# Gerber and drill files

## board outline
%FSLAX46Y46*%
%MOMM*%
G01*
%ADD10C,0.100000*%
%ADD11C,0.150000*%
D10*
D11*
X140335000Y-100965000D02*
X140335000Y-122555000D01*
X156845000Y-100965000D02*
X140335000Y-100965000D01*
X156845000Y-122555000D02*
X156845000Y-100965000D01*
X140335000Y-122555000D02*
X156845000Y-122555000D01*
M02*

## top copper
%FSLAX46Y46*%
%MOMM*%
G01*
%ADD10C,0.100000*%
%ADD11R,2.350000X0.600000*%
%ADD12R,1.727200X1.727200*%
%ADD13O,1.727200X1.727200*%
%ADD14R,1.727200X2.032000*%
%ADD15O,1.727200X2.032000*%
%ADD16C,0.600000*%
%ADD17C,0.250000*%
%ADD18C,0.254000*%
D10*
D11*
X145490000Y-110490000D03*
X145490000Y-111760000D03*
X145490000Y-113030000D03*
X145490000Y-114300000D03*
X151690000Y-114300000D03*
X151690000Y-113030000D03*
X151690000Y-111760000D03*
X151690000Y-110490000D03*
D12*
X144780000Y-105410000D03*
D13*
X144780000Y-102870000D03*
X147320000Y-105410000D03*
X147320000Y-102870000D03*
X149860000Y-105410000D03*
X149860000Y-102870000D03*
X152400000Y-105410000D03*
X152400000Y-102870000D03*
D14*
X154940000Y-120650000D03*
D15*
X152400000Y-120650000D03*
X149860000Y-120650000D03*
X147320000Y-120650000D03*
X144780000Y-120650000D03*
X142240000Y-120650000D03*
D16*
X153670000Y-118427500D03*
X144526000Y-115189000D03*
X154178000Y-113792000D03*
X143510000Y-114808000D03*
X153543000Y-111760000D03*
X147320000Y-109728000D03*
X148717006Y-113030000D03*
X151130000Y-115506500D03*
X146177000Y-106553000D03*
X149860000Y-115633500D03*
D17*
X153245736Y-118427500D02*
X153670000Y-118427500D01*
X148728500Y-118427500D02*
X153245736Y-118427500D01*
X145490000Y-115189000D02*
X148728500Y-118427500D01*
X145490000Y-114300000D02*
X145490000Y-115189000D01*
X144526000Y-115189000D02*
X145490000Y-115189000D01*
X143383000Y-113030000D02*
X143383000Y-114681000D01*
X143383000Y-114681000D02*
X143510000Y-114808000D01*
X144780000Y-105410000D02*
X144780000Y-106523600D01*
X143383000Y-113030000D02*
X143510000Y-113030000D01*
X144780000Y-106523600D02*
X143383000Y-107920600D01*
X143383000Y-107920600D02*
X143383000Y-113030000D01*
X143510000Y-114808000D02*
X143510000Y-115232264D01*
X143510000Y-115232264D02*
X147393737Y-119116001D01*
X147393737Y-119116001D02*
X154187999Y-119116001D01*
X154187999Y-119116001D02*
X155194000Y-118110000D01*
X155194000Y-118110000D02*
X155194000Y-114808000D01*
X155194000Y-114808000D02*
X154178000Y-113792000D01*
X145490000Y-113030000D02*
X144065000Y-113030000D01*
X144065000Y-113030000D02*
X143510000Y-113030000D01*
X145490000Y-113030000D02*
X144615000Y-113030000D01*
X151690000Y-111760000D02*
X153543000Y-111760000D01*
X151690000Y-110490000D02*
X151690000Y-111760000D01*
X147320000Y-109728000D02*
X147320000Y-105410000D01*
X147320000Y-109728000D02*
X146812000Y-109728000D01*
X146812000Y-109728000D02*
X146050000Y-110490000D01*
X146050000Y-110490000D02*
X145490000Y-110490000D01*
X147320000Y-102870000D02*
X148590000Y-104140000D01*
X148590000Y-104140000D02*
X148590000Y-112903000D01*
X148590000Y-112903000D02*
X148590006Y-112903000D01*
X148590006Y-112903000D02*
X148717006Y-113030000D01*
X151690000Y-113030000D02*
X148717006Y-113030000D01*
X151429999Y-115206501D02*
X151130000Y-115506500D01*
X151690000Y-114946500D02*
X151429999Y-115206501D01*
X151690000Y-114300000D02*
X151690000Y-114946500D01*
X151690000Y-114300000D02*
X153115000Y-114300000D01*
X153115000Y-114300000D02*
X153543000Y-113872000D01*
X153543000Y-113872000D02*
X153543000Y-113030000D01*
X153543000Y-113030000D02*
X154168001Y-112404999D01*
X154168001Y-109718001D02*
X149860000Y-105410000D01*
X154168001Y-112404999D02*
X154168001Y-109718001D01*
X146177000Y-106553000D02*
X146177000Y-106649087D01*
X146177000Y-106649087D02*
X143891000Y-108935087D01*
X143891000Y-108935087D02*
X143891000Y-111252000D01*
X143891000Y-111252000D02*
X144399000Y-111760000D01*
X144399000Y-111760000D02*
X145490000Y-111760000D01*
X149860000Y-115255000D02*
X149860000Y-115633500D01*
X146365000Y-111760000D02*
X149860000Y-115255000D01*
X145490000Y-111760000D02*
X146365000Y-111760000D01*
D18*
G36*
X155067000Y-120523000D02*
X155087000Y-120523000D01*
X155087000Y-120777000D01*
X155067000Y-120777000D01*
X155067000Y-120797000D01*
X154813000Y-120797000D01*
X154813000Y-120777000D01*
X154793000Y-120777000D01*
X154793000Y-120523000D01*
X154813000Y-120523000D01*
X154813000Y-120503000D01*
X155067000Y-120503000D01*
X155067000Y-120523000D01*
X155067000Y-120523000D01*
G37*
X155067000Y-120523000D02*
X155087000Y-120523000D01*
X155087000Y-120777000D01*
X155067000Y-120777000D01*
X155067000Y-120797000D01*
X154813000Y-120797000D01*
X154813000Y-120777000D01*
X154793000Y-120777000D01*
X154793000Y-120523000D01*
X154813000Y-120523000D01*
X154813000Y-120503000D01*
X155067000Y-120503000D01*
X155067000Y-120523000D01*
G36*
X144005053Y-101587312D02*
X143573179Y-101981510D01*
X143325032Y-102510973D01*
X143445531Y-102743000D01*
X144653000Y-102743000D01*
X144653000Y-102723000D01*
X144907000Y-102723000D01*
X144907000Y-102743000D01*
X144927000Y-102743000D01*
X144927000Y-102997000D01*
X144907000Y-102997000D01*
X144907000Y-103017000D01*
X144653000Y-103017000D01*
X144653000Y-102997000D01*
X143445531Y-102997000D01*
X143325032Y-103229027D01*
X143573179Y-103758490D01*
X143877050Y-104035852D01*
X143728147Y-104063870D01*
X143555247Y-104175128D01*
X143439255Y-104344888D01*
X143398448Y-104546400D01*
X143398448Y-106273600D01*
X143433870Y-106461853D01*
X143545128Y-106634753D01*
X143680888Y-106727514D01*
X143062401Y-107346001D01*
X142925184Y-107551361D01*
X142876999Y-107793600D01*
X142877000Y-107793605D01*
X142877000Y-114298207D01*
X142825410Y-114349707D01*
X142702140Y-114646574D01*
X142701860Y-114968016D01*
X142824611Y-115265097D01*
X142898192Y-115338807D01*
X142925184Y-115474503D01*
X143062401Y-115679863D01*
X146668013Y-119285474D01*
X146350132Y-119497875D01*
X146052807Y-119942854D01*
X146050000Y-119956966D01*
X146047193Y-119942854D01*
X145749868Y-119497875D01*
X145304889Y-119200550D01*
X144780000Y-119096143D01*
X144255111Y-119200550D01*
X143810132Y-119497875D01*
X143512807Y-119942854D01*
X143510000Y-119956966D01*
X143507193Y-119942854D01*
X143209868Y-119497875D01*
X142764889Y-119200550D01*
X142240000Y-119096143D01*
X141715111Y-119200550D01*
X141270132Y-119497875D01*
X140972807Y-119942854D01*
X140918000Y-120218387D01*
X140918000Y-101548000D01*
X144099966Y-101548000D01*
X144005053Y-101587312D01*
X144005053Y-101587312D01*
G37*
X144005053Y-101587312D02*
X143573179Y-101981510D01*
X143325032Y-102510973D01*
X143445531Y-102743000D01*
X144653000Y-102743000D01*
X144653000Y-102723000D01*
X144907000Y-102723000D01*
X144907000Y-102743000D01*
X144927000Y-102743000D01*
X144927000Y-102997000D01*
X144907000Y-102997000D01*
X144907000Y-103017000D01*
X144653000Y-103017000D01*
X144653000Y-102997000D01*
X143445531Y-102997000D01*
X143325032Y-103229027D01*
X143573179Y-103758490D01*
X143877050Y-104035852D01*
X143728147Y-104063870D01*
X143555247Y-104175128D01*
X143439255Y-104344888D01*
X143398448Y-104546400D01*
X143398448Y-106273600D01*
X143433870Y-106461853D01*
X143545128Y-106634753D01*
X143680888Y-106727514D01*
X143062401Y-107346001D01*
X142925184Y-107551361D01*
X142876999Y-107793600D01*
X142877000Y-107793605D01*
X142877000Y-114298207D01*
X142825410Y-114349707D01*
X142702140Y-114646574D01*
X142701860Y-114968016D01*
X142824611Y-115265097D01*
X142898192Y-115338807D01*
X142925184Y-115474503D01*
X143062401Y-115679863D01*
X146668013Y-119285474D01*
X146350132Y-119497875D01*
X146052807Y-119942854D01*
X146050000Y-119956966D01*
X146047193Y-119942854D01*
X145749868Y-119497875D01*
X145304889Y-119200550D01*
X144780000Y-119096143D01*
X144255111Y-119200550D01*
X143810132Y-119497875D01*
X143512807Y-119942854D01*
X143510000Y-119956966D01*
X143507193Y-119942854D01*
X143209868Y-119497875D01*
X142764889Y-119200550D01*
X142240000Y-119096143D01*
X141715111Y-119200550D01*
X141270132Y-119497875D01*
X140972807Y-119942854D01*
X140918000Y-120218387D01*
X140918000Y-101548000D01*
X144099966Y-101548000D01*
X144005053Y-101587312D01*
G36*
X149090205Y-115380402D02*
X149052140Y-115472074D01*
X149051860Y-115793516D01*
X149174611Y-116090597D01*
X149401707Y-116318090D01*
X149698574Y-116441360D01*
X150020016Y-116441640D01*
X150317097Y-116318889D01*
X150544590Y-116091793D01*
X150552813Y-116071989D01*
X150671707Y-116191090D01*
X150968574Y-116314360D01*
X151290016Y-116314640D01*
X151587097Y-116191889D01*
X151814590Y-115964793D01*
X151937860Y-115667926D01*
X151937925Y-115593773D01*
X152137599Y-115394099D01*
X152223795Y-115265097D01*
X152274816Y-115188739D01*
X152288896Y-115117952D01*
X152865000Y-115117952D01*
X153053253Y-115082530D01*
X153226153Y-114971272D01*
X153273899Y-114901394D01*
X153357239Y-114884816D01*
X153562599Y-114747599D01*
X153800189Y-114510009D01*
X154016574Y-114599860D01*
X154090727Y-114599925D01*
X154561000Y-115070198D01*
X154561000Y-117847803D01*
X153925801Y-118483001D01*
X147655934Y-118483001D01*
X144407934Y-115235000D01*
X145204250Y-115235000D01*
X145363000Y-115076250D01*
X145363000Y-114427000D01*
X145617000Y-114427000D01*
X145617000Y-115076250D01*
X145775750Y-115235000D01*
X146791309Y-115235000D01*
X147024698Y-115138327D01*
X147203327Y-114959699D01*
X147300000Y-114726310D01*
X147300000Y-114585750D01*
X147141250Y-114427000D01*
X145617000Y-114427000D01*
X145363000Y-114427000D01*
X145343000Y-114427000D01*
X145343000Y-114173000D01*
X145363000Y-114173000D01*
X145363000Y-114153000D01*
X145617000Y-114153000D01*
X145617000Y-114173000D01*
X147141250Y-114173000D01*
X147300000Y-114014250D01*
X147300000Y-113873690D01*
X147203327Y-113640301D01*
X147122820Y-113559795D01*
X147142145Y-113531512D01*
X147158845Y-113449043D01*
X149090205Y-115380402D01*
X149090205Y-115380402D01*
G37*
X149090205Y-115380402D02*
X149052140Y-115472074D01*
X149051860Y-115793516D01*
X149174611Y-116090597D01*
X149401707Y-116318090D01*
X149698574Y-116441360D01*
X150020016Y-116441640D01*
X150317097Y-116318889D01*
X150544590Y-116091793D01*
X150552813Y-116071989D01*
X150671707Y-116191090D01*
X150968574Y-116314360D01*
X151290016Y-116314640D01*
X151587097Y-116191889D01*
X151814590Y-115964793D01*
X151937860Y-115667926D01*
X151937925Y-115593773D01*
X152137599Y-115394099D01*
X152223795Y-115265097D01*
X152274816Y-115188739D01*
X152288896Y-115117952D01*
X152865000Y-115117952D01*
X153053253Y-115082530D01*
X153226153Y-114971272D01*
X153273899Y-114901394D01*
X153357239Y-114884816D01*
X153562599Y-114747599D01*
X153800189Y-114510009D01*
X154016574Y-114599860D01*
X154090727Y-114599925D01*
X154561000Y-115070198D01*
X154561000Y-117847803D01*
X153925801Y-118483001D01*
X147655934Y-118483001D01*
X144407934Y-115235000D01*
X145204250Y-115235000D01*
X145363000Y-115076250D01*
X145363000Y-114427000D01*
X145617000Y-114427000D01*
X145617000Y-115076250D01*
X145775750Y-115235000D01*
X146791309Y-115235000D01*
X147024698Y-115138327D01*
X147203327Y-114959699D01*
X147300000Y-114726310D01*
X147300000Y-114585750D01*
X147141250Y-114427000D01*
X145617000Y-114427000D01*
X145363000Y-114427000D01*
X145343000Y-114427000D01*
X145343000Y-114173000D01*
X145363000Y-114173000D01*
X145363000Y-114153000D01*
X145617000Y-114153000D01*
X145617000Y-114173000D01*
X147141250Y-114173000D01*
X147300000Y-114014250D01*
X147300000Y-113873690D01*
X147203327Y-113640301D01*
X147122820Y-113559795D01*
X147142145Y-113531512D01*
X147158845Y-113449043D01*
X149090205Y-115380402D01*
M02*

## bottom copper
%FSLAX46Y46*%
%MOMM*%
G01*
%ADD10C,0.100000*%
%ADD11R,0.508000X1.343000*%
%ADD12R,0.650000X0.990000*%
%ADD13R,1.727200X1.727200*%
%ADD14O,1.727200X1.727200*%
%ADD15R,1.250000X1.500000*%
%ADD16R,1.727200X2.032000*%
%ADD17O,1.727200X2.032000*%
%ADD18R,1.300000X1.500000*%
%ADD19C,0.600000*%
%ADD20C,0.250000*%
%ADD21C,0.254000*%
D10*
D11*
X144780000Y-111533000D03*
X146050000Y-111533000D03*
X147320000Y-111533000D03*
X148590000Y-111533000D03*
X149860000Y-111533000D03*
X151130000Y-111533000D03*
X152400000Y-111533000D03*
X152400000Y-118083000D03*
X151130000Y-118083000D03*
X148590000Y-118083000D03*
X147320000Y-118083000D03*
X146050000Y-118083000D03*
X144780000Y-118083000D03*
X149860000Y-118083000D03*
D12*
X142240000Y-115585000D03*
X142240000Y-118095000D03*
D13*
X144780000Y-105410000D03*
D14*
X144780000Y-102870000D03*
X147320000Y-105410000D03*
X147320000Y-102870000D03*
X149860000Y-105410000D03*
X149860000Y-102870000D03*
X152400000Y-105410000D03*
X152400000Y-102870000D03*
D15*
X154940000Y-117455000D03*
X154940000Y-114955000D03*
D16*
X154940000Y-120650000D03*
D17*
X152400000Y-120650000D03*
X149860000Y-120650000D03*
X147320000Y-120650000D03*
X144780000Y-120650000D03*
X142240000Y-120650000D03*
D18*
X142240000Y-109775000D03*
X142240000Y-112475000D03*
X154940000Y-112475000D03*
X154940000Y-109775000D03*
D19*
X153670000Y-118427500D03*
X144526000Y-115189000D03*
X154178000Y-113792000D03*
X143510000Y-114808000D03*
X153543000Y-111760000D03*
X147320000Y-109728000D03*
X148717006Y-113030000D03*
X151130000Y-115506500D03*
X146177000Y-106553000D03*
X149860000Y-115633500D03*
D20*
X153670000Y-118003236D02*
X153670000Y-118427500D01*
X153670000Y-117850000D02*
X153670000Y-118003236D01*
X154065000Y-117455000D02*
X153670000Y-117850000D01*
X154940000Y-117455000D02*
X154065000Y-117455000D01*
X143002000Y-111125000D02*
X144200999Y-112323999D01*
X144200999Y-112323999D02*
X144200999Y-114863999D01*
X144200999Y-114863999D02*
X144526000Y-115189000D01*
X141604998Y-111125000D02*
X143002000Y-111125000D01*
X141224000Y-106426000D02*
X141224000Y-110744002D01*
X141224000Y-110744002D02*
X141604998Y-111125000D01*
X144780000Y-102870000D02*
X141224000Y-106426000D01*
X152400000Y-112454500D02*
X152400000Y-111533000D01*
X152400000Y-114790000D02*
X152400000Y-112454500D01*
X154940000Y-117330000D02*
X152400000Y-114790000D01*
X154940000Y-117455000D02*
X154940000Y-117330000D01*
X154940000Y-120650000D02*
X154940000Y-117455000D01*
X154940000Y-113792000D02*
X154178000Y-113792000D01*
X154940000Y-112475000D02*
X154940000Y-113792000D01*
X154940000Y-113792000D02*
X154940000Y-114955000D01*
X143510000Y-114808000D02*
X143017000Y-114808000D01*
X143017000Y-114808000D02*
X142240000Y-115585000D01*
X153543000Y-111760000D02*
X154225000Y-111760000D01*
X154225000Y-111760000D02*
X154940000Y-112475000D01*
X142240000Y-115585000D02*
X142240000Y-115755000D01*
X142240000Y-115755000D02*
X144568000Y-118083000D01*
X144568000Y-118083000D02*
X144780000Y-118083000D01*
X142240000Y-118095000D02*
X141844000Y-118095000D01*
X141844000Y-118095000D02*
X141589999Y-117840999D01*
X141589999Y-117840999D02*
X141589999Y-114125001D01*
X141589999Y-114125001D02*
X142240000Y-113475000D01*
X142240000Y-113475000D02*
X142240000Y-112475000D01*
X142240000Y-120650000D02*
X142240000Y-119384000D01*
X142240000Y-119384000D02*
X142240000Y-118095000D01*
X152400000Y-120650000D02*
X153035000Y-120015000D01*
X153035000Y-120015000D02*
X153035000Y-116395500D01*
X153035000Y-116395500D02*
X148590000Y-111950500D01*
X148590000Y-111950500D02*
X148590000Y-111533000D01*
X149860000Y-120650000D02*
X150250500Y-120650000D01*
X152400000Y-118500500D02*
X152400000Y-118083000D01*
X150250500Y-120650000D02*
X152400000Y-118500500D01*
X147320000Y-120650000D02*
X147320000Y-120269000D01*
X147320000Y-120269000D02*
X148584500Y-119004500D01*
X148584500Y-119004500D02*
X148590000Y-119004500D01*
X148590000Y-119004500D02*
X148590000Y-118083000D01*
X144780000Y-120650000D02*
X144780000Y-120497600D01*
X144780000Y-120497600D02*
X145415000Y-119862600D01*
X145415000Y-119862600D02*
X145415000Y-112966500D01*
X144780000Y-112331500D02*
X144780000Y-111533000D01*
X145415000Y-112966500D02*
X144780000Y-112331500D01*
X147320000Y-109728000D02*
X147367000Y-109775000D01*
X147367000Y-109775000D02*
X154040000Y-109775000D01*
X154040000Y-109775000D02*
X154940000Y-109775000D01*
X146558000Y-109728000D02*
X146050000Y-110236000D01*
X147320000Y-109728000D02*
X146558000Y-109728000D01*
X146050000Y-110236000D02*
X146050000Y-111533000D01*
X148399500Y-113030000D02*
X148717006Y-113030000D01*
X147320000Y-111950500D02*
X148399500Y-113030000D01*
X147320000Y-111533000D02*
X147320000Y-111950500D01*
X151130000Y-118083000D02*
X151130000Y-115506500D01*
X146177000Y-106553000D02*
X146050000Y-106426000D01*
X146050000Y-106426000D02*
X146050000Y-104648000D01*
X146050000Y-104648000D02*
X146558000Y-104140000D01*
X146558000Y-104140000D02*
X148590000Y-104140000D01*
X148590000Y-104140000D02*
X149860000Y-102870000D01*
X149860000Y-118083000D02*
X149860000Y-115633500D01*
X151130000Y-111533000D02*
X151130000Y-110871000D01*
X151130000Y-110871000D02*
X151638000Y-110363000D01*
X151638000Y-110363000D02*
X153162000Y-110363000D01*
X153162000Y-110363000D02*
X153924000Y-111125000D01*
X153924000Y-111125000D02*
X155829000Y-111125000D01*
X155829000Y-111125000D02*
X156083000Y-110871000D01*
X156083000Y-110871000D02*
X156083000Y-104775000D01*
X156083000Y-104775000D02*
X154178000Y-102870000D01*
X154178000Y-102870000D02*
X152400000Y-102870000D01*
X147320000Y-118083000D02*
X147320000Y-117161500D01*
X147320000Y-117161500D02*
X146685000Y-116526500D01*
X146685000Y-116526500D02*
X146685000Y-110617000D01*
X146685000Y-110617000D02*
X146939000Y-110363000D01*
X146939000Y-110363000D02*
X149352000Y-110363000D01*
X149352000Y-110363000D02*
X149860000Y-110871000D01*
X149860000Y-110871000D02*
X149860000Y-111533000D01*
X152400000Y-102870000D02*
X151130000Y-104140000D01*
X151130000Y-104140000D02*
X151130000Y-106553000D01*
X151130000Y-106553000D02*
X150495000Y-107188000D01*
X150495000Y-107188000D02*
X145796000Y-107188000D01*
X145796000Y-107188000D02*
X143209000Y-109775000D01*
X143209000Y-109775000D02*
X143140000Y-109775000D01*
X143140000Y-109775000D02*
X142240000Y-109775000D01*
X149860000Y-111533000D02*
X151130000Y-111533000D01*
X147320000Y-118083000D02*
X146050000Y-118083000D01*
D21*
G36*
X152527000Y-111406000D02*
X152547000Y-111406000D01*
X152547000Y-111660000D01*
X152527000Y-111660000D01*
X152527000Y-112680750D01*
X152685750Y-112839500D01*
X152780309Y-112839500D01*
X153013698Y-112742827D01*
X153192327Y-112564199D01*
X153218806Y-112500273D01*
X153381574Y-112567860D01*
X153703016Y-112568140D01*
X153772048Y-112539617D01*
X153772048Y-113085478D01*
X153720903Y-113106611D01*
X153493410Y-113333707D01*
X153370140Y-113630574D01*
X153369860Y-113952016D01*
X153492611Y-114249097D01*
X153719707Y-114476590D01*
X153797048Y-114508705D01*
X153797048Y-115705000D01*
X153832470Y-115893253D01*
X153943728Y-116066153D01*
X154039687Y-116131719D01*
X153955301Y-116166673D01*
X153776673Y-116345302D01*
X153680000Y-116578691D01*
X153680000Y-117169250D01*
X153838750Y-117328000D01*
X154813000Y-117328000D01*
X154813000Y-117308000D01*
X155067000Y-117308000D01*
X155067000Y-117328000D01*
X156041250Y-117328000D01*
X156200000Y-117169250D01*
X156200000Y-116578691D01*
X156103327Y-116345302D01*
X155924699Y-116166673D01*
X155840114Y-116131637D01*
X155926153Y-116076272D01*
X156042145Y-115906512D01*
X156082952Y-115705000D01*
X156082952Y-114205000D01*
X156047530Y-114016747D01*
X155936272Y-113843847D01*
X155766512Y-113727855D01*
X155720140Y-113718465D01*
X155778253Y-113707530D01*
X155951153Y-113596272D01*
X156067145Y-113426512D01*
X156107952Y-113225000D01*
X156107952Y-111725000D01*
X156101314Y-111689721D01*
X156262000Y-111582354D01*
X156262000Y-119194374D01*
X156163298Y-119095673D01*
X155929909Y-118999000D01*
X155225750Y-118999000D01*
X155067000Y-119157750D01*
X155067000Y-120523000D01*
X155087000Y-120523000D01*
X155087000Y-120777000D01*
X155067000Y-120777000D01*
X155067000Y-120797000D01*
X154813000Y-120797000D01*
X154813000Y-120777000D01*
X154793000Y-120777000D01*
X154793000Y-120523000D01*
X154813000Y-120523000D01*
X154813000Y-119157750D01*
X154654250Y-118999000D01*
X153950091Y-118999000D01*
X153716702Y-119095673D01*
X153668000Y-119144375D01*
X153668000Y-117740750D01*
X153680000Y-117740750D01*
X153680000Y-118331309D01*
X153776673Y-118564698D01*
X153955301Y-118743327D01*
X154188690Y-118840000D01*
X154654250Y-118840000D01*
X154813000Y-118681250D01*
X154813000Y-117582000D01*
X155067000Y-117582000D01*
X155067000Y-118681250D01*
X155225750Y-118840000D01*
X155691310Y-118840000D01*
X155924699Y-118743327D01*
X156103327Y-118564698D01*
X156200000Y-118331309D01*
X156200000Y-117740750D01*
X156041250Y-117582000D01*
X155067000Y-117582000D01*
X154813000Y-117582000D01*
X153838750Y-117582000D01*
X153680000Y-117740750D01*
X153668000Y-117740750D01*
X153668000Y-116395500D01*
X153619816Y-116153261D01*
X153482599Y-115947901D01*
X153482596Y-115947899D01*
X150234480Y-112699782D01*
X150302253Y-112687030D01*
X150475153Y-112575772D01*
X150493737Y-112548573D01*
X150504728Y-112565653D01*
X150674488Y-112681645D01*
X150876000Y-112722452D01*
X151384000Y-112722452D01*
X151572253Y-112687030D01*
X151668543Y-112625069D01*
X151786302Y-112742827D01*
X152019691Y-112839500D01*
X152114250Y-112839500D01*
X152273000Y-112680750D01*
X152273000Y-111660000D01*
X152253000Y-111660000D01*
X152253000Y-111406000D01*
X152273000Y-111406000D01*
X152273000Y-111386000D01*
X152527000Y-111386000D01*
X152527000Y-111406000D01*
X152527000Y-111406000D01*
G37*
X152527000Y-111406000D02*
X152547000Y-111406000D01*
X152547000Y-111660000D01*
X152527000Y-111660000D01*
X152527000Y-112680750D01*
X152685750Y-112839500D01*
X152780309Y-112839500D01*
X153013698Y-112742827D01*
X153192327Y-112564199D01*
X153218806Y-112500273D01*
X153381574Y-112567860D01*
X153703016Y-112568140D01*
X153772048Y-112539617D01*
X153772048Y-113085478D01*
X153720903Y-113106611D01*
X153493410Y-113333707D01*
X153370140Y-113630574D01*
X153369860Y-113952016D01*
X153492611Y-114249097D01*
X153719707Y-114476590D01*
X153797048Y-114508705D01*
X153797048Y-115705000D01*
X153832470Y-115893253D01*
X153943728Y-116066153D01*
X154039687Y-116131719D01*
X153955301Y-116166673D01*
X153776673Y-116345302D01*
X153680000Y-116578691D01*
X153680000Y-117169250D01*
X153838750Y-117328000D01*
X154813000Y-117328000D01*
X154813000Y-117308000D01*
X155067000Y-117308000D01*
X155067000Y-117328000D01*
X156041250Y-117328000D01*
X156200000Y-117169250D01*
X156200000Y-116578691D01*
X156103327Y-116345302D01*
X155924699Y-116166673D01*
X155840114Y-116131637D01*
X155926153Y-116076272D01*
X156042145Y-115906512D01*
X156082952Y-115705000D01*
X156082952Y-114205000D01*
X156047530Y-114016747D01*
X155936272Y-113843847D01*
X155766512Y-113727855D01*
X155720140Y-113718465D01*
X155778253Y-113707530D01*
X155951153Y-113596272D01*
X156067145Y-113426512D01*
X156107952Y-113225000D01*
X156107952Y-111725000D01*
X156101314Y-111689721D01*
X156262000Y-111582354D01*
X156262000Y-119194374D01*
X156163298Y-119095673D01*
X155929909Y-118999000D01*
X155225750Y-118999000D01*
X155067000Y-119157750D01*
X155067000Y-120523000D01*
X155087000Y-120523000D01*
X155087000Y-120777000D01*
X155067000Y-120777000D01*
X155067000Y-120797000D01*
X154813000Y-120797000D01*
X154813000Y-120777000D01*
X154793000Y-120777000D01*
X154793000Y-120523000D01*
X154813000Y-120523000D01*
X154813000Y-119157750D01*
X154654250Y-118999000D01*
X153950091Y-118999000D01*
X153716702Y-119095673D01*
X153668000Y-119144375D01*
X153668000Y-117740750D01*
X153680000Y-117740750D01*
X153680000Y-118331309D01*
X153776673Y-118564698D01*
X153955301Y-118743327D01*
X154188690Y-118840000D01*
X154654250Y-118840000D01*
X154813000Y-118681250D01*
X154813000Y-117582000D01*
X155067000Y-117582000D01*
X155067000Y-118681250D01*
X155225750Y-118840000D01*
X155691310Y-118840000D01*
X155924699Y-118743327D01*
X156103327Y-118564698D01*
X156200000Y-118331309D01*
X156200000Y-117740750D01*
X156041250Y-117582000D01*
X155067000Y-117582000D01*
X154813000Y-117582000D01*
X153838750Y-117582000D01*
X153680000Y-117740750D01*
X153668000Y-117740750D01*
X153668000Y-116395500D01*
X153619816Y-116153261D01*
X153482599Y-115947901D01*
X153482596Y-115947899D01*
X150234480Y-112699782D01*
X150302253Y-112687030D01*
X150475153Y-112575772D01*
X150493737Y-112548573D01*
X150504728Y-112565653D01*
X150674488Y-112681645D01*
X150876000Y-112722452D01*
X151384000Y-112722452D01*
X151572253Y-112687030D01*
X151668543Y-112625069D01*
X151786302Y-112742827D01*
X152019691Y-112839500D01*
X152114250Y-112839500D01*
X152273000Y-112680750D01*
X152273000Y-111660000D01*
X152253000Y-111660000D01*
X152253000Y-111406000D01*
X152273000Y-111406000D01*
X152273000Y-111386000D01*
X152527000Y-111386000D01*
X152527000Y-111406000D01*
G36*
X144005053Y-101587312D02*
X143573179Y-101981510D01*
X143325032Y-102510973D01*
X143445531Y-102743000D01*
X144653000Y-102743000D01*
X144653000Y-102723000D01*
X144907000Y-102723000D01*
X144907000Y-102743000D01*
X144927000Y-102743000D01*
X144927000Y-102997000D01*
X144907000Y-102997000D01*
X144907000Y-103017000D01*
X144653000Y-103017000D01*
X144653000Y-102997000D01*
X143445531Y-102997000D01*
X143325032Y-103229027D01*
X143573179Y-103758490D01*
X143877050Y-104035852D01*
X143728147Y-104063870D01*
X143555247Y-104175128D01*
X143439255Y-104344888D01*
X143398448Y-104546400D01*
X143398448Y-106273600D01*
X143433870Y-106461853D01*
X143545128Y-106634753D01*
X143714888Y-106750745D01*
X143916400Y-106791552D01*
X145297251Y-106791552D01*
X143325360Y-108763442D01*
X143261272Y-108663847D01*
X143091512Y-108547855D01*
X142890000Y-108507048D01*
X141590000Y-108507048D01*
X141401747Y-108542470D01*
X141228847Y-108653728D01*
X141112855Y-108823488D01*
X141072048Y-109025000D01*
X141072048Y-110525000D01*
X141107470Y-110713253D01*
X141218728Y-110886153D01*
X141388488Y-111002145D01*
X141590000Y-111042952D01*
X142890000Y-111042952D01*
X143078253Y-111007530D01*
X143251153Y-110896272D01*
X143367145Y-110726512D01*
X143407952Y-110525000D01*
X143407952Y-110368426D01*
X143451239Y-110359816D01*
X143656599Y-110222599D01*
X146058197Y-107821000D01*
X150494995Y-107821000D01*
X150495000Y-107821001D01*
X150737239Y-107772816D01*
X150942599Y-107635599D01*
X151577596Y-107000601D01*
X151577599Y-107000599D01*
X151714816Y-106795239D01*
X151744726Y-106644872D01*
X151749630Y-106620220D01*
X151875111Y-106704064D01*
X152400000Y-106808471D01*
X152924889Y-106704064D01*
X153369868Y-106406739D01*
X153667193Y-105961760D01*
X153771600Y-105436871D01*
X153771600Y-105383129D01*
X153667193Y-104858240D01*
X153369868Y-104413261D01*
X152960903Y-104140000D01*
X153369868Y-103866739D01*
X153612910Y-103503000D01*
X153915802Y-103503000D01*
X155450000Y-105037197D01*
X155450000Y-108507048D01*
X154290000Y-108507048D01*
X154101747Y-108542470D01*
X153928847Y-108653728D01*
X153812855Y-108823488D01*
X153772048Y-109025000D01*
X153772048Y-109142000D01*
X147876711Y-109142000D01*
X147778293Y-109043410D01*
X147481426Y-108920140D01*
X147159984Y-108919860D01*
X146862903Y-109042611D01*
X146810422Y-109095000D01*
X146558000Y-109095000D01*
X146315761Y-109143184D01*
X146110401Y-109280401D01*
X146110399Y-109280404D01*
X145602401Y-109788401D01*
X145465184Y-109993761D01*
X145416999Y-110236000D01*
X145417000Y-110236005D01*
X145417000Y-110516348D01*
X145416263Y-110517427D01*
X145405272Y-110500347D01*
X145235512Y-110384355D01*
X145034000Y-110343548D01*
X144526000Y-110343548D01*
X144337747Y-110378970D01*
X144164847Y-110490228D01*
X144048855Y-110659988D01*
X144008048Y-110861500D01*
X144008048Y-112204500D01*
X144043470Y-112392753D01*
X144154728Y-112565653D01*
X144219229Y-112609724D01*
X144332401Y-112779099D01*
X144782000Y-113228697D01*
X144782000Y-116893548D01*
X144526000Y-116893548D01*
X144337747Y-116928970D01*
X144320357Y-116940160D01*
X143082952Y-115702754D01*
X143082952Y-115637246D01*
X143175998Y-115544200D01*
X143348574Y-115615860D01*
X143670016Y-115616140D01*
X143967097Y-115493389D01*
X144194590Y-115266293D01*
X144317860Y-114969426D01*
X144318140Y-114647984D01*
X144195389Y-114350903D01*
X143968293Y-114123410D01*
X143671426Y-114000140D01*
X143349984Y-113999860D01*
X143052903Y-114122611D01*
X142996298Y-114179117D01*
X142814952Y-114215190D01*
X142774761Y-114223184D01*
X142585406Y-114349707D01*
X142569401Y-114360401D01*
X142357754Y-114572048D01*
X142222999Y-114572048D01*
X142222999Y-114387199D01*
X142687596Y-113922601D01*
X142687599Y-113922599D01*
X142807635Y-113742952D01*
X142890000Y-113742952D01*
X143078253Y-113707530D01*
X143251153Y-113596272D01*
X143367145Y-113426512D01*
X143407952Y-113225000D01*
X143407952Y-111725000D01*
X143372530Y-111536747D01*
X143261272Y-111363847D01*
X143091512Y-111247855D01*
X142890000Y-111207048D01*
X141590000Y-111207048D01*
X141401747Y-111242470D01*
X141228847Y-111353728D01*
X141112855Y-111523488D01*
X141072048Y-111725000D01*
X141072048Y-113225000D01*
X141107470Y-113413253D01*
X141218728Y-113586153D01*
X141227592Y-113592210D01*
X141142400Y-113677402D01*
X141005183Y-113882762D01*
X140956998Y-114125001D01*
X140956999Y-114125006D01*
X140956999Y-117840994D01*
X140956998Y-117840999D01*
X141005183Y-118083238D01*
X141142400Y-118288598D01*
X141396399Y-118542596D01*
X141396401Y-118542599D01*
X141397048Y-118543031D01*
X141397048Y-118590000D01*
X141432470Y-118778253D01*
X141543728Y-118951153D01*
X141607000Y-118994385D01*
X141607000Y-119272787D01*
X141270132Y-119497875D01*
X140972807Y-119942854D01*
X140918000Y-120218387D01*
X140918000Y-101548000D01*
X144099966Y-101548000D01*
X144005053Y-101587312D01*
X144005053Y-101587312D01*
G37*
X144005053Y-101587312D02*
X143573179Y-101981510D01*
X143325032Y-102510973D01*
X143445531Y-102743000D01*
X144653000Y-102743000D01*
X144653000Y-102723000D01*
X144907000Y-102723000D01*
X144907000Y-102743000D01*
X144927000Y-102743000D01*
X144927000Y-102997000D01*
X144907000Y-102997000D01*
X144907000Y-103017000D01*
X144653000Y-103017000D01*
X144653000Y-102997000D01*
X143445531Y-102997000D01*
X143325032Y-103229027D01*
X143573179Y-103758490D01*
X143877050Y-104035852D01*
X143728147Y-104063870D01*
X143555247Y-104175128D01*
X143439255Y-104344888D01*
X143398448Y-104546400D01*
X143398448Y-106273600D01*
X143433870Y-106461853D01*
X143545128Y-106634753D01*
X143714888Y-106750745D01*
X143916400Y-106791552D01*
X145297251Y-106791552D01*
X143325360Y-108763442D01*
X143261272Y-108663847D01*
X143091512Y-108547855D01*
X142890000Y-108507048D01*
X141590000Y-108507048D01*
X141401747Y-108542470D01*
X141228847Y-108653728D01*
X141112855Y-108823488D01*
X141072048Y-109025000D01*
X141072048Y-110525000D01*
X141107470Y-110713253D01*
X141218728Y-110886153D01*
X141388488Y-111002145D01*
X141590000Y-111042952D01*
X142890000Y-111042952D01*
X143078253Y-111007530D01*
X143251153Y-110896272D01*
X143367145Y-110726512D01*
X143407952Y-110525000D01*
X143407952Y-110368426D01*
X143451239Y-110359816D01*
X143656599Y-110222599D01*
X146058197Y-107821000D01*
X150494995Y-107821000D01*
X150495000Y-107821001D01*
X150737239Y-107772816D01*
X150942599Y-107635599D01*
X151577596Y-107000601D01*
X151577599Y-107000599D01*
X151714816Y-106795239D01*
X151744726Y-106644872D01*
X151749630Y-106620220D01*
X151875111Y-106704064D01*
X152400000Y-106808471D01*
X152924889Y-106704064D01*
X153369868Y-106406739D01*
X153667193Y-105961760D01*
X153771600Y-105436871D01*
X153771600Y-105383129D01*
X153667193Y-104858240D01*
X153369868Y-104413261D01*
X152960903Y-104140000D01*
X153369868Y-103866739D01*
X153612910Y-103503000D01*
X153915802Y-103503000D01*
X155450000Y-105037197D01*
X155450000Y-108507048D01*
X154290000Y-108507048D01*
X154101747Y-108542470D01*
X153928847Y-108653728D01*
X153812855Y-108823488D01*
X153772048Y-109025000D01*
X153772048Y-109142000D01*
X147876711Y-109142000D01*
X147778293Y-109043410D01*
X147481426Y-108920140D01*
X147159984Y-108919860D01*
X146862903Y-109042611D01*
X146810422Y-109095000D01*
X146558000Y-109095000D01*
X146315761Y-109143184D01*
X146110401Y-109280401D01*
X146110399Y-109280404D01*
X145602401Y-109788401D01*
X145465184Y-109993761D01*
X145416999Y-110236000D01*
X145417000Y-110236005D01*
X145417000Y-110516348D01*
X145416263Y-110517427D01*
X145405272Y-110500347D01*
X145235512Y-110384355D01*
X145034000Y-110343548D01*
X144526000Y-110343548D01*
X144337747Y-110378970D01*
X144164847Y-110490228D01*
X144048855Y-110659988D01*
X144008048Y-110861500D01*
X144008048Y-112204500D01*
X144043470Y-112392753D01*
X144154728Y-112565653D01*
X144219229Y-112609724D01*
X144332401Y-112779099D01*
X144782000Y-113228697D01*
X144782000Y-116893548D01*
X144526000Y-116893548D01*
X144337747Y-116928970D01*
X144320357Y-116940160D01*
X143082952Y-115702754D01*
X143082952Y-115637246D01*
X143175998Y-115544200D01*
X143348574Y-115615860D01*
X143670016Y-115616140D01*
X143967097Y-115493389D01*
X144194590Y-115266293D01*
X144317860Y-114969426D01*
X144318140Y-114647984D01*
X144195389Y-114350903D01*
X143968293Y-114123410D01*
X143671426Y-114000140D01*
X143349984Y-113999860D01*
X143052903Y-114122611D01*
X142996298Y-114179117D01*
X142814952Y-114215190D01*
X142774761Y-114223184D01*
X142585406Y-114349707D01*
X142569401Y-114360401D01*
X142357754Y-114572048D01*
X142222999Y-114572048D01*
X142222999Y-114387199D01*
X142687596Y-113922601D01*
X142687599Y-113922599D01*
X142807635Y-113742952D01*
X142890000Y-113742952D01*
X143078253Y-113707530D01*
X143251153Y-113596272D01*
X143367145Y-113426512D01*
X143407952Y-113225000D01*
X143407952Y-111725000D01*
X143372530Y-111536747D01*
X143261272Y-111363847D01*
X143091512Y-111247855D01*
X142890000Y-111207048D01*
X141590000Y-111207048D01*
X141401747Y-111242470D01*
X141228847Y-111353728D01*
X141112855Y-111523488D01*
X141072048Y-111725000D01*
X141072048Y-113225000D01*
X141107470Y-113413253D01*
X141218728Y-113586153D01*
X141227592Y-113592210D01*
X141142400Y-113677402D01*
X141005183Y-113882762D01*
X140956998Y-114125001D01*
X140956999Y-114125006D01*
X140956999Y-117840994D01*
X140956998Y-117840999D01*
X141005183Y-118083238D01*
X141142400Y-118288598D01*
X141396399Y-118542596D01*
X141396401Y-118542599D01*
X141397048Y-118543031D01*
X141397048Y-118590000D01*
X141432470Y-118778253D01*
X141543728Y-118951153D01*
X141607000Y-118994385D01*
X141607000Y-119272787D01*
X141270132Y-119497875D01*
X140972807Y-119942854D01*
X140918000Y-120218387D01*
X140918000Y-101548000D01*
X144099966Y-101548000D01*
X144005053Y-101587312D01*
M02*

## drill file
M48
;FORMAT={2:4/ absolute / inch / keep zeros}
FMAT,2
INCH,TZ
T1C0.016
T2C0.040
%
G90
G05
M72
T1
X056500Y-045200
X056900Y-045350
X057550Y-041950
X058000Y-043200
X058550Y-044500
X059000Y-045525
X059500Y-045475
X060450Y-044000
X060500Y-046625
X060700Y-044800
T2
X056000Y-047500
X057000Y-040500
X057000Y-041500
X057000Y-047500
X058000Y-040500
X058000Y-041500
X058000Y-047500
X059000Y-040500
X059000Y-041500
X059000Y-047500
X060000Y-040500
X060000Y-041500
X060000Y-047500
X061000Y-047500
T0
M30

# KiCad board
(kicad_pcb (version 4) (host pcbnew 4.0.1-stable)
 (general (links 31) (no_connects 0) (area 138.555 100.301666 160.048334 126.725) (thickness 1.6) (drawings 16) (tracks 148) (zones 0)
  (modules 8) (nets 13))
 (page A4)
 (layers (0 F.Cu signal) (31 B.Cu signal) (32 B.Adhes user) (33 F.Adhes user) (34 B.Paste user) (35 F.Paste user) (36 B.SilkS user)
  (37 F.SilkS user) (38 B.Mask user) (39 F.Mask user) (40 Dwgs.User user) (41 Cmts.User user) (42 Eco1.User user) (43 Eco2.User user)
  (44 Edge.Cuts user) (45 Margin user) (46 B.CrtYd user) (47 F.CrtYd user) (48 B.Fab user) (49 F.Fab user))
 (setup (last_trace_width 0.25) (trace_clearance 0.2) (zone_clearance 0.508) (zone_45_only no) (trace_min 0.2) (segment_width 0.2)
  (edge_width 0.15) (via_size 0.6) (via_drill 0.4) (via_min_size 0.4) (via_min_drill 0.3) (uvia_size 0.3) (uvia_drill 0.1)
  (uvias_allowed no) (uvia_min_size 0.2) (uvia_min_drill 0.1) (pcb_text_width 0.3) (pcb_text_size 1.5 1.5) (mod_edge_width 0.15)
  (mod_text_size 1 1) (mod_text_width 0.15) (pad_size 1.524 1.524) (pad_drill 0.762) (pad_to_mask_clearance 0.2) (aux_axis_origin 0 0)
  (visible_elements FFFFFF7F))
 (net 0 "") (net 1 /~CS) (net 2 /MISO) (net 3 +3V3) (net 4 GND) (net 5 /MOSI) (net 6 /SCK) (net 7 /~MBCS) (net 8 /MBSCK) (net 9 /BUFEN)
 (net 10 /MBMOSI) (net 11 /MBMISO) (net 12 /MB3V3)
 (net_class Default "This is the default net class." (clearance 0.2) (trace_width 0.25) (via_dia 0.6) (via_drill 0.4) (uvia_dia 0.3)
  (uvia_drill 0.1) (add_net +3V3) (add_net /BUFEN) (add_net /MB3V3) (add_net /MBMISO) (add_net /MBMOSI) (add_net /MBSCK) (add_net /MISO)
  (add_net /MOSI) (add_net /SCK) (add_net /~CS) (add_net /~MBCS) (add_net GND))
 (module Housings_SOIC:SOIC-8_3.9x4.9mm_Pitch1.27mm (layer F.Cu) (at 148.59 112.395)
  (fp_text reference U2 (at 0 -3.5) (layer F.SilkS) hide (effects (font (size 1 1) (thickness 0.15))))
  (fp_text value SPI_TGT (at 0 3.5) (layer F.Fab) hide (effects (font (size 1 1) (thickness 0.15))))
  (pad 1 smd rect (at -3.1 -1.905) (size 2.35 0.6) (layers F.Cu F.Paste F.Mask) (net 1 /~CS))
  (pad 2 smd rect (at -3.1 -0.635) (size 2.35 0.6) (layers F.Cu F.Paste F.Mask) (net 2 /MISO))
  (pad 3 smd rect (at -3.1 0.635) (size 2.35 0.6) (layers F.Cu F.Paste F.Mask) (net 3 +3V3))
  (pad 4 smd rect (at -3.1 1.905) (size 2.35 0.6) (layers F.Cu F.Paste F.Mask) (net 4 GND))
  (pad 5 smd rect (at 3.1 1.905) (size 2.35 0.6) (layers F.Cu F.Paste F.Mask) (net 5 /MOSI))
  (pad 6 smd rect (at 3.1 0.635) (size 2.35 0.6) (layers F.Cu F.Paste F.Mask) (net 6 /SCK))
  (pad 7 smd rect (at 3.1 -0.635) (size 2.35 0.6) (layers F.Cu F.Paste F.Mask) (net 3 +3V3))
  (pad 8 smd rect (at 3.1 -1.905) (size 2.35 0.6) (layers F.Cu F.Paste F.Mask) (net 3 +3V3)))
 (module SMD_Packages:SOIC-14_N (layer B.Cu) (at 148.59 114.935)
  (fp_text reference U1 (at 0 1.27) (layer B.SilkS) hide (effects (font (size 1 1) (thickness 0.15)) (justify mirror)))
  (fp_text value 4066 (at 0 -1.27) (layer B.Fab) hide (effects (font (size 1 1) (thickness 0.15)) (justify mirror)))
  (pad 1 smd rect (at -3.81 -3.402) (size 0.508 1.343) (layers B.Cu B.Paste B.Mask) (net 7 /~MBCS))
  (pad 2 smd rect (at -2.54 -3.402) (size 0.508 1.343) (layers B.Cu B.Paste B.Mask) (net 1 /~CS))
  (pad 3 smd rect (at -1.27 -3.402) (size 0.508 1.343) (layers B.Cu B.Paste B.Mask) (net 6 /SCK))
  (pad 4 smd rect (at 0 -3.402) (size 0.508 1.343) (layers B.Cu B.Paste B.Mask) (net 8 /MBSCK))
  (pad 5 smd rect (at 1.27 -3.402) (size 0.508 1.343) (layers B.Cu B.Paste B.Mask) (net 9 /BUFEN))
  (pad 6 smd rect (at 2.54 -3.402) (size 0.508 1.343) (layers B.Cu B.Paste B.Mask) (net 9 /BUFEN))
  (pad 7 smd rect (at 3.81 -3.402) (size 0.508 1.343) (layers B.Cu B.Paste B.Mask) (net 4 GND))
  (pad 8 smd rect (at 3.81 3.148) (size 0.508 1.343) (layers B.Cu B.Paste B.Mask) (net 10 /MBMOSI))
  (pad 9 smd rect (at 2.54 3.148) (size 0.508 1.343) (layers B.Cu B.Paste B.Mask) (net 5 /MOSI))
  (pad 11 smd rect (at 0 3.148) (size 0.508 1.343) (layers B.Cu B.Paste B.Mask) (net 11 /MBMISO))
  (pad 12 smd rect (at -1.27 3.148) (size 0.508 1.343) (layers B.Cu B.Paste B.Mask) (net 9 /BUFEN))
  (pad 13 smd rect (at -2.54 3.148) (size 0.508 1.343) (layers B.Cu B.Paste B.Mask) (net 9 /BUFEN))
  (pad 14 smd rect (at -3.81 3.148) (size 0.508 1.343) (layers B.Cu B.Paste B.Mask) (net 3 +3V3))
  (pad 10 smd rect (at 1.27 3.148 180) (size 0.508 1.343) (layers B.Cu B.Paste B.Mask) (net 2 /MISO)))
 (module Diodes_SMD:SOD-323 (layer B.Cu) (at 142.24 116.84 270)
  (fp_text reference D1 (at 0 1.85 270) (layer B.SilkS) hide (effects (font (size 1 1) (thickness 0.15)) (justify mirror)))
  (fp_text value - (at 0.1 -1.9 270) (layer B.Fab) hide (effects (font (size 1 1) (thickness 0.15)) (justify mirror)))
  (pad 1 smd rect (at -1.255 0 270) (size 0.99 0.65) (layers B.Cu B.Paste B.Mask) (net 3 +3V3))
  (pad 2 smd rect (at 1.255 0 270) (size 0.99 0.65) (layers B.Cu B.Paste B.Mask) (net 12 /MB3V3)))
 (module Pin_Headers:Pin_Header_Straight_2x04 (layer F.Cu) (at 144.78 105.41 90)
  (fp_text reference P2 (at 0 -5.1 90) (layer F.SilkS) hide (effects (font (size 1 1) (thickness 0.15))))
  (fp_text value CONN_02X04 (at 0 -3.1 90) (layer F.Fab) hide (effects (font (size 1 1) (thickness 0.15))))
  (pad 1 thru_hole rect (at 0 0 90) (size 1.7272 1.7272) (drill 1.016) (layers *.Cu *.Mask F.SilkS) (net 3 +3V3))
  (pad 2 thru_hole oval (at 2.54 0 90) (size 1.7272 1.7272) (drill 1.016) (layers *.Cu *.Mask F.SilkS) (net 4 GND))
  (pad 3 thru_hole oval (at 0 2.54 90) (size 1.7272 1.7272) (drill 1.016) (layers *.Cu *.Mask F.SilkS) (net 1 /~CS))
  (pad 4 thru_hole oval (at 2.54 2.54 90) (size 1.7272 1.7272) (drill 1.016) (layers *.Cu *.Mask F.SilkS) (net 6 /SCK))
  (pad 5 thru_hole oval (at 0 5.08 90) (size 1.7272 1.7272) (drill 1.016) (layers *.Cu *.Mask F.SilkS) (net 5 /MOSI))
  (pad 6 thru_hole oval (at 2.54 5.08 90) (size 1.7272 1.7272) (drill 1.016) (layers *.Cu *.Mask F.SilkS) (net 2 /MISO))
  (pad 7 thru_hole oval (at 0 7.62 90) (size 1.7272 1.7272) (drill 1.016) (layers *.Cu *.Mask F.SilkS))
  (pad 8 thru_hole oval (at 2.54 7.62 90) (size 1.7272 1.7272) (drill 1.016) (layers *.Cu *.Mask F.SilkS) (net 9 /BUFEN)))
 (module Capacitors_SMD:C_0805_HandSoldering (layer B.Cu) (at 154.94 116.205 90)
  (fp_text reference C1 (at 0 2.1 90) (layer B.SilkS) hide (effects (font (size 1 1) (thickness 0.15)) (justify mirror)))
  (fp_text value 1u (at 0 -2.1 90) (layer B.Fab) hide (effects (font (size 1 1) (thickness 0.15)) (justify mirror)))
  (pad 1 smd rect (at -1.25 0 90) (size 1.5 1.25) (layers B.Cu B.Paste B.Mask) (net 4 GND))
  (pad 2 smd rect (at 1.25 0 90) (size 1.5 1.25) (layers B.Cu B.Paste B.Mask) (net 3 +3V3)))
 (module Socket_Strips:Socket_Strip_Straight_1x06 (layer F.Cu) (at 154.94 120.65 180)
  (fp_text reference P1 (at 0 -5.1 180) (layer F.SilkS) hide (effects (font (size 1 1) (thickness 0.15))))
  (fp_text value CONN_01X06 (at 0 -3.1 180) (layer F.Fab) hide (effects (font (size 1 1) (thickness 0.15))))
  (pad 1 thru_hole rect (at 0 0 180) (size 1.7272 2.032) (drill 1.016) (layers *.Cu *.Mask F.SilkS) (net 4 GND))
  (pad 2 thru_hole oval (at 2.54 0 180) (size 1.7272 2.032) (drill 1.016) (layers *.Cu *.Mask F.SilkS) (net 8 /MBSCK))
  (pad 3 thru_hole oval (at 5.08 0 180) (size 1.7272 2.032) (drill 1.016) (layers *.Cu *.Mask F.SilkS) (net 10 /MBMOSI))
  (pad 4 thru_hole oval (at 7.62 0 180) (size 1.7272 2.032) (drill 1.016) (layers *.Cu *.Mask F.SilkS) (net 11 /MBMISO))
  (pad 5 thru_hole oval (at 10.16 0 180) (size 1.7272 2.032) (drill 1.016) (layers *.Cu *.Mask F.SilkS) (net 7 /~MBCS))
  (pad 6 thru_hole oval (at 12.7 0 180) (size 1.7272 2.032) (drill 1.016) (layers *.Cu *.Mask F.SilkS) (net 12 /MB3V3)))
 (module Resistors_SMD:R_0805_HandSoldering (layer B.Cu) (at 142.24 111.125 270)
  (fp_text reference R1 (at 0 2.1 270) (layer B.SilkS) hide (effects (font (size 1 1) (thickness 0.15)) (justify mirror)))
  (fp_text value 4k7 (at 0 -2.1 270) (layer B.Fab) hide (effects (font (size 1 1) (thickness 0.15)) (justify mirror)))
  (pad 1 smd rect (at -1.35 0 270) (size 1.5 1.3) (layers B.Cu B.Paste B.Mask) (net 9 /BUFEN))
  (pad 2 smd rect (at 1.35 0 270) (size 1.5 1.3) (layers B.Cu B.Paste B.Mask) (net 12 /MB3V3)))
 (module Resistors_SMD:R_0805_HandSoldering (layer B.Cu) (at 154.94 111.125 90)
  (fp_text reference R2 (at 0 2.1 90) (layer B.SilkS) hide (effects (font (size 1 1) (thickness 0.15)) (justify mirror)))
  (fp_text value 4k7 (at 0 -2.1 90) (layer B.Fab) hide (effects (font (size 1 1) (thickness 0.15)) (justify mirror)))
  (pad 1 smd rect (at -1.35 0 90) (size 1.5 1.3) (layers B.Cu B.Paste B.Mask) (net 3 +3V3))
  (pad 2 smd rect (at 1.35 0 90) (size 1.5 1.3) (layers B.Cu B.Paste B.Mask) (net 1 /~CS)))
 (gr_line (start 140.335 100.965) (end 140.335 122.555) (layer Edge.Cuts) (width 0.15))
 (gr_line (start 156.845 100.965) (end 140.335 100.965) (layer Edge.Cuts) (width 0.15))
 (gr_line (start 156.845 122.555) (end 156.845 100.965) (layer Edge.Cuts) (width 0.15))
 (gr_line (start 140.335 122.555) (end 156.845 122.555) (angle 90) (layer Edge.Cuts) (width 0.15))
 (segment (start 153.245736 118.4275) (end 153.67 118.4275) (width 0.25) (layer F.Cu) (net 4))
 (segment (start 153.67 118.003236) (end 153.67 118.4275) (width 0.25) (layer B.Cu) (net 4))
 (segment (start 153.67 117.85) (end 153.67 118.003236) (width 0.25) (layer B.Cu) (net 4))
 (segment (start 154.065 117.455) (end 153.67 117.85) (width 0.25) (layer B.Cu) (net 4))
 (via (at 153.67 118.4275) (size 0.6) (drill 0.4) (layers F.Cu B.Cu) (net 4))
 (segment (start 148.7285 118.4275) (end 153.245736 118.4275) (width 0.25) (layer F.Cu) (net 4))
 (segment (start 145.49 115.189) (end 148.7285 118.4275) (width 0.25) (layer F.Cu) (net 4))
 (segment (start 154.94 117.455) (end 154.065 117.455) (width 0.25) (layer B.Cu) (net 4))
 (segment (start 145.49 114.3) (end 145.49 115.189) (width 0.25) (layer F.Cu) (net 4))
 (segment (start 144.526 115.189) (end 145.49 115.189) (width 0.25) (layer F.Cu) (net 4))
 (segment (start 143.002 111.125) (end 144.200999 112.323999) (width 0.25) (layer B.Cu) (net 4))
 (segment (start 144.200999 112.323999) (end 144.200999 114.863999) (width 0.25) (layer B.Cu) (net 4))
 (segment (start 144.200999 114.863999) (end 144.526 115.189) (width 0.25) (layer B.Cu) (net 4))
 (via (at 144.526 115.189) (size 0.6) (drill 0.4) (layers F.Cu B.Cu) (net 4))
 (segment (start 141.604998 111.125) (end 143.002 111.125) (width 0.25) (layer B.Cu) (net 4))
 (segment (start 141.224 106.426) (end 141.224 110.744002) (width 0.25) (layer B.Cu) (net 4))
 (segment (start 141.224 110.744002) (end 141.604998 111.125) (width 0.25) (layer B.Cu) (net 4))
 (segment (start 144.78 102.87) (end 141.224 106.426) (width 0.25) (layer B.Cu) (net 4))
 (segment (start 152.4 112.4545) (end 152.4 111.533) (width 0.25) (layer B.Cu) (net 4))
 (segment (start 152.4 114.79) (end 152.4 112.4545) (width 0.25) (layer B.Cu) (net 4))
 (segment (start 154.94 117.33) (end 152.4 114.79) (width 0.25) (layer B.Cu) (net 4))
 (segment (start 154.94 117.455) (end 154.94 117.33) (width 0.25) (layer B.Cu) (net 4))
 (segment (start 154.94 120.65) (end 154.94 117.455) (width 0.25) (layer B.Cu) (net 4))
 (segment (start 143.383 113.03) (end 143.383 114.681) (width 0.25) (layer F.Cu) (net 3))
 (segment (start 143.383 114.681) (end 143.51 114.808) (width 0.25) (layer F.Cu) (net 3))
 (segment (start 144.78 105.41) (end 144.78 106.5236) (width 0.25) (layer F.Cu) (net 3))
 (segment (start 143.383 113.03) (end 143.51 113.03) (width 0.25) (layer F.Cu) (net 3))
 (segment (start 144.78 106.5236) (end 143.383 107.9206) (width 0.25) (layer F.Cu) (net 3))
 (segment (start 143.383 107.9206) (end 143.383 113.03) (width 0.25) (layer F.Cu) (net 3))
 (segment (start 143.51 114.808) (end 143.51 115.232264) (width 0.25) (layer F.Cu) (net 3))
 (segment (start 143.51 115.232264) (end 147.393737 119.116001) (width 0.25) (layer F.Cu) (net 3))
 (segment (start 147.393737 119.116001) (end 154.187999 119.116001) (width 0.25) (layer F.Cu) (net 3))
 (segment (start 154.187999 119.116001) (end 155.194 118.11) (width 0.25) (layer F.Cu) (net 3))
 (segment (start 155.194 118.11) (end 155.194 114.808) (width 0.25) (layer F.Cu) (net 3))
 (segment (start 155.194 114.808) (end 154.178 113.792) (width 0.25) (layer F.Cu) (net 3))
 (via (at 154.178 113.792) (size 0.6) (drill 0.4) (layers F.Cu B.Cu) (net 3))
 (segment (start 154.94 113.792) (end 154.178 113.792) (width 0.25) (layer B.Cu) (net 3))
 (segment (start 154.94 112.475) (end 154.94 113.792) (width 0.25) (layer B.Cu) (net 3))
 (segment (start 154.94 113.792) (end 154.94 114.955) (width 0.25) (layer B.Cu) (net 3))
 (segment (start 145.49 113.03) (end 144.065 113.03) (width 0.25) (layer F.Cu) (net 3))
 (segment (start 144.065 113.03) (end 143.51 113.03) (width 0.25) (layer F.Cu) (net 3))
 (segment (start 143.51 114.808) (end 143.017 114.808) (width 0.25) (layer B.Cu) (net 3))
 (segment (start 143.017 114.808) (end 142.24 115.585) (width 0.25) (layer B.Cu) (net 3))
 (segment (start 145.49 113.03) (end 144.615 113.03) (width 0.25) (layer F.Cu) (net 3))
 (via (at 143.51 114.808) (size 0.6) (drill 0.4) (layers F.Cu B.Cu) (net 3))
 (segment (start 153.543 111.76) (end 154.225 111.76) (width 0.25) (layer B.Cu) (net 3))
 (segment (start 154.225 111.76) (end 154.94 112.475) (width 0.25) (layer B.Cu) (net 3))
 (segment (start 151.69 111.76) (end 153.543 111.76) (width 0.25) (layer F.Cu) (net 3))
 (via (at 153.543 111.76) (size 0.6) (drill 0.4) (layers F.Cu B.Cu) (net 3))
 (segment (start 151.69 110.49) (end 151.69 111.76) (width 0.25) (layer F.Cu) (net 3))
 (segment (start 142.24 115.585) (end 142.24 115.755) (width 0.25) (layer B.Cu) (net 3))
 (segment (start 142.24 115.755) (end 144.568 118.083) (width 0.25) (layer B.Cu) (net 3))
 (segment (start 144.568 118.083) (end 144.78 118.083) (width 0.25) (layer B.Cu) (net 3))
 (segment (start 142.24 118.095) (end 141.844 118.095) (width 0.25) (layer B.Cu) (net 12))
 (segment (start 141.844 118.095) (end 141.589999 117.840999) (width 0.25) (layer B.Cu) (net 12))
 (segment (start 141.589999 117.840999) (end 141.589999 114.125001) (width 0.25) (layer B.Cu) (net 12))
 (segment (start 141.589999 114.125001) (end 142.24 113.475) (width 0.25) (layer B.Cu) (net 12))
 (segment (start 142.24 113.475) (end 142.24 112.475) (width 0.25) (layer B.Cu) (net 12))
 (segment (start 142.24 120.65) (end 142.24 119.384) (width 0.25) (layer B.Cu) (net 12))
 (segment (start 142.24 119.384) (end 142.24 118.095) (width 0.25) (layer B.Cu) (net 12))
 (segment (start 152.4 120.65) (end 153.035 120.015) (width 0.25) (layer B.Cu) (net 8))
 (segment (start 153.035 120.015) (end 153.035 116.3955) (width 0.25) (layer B.Cu) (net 8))
 (segment (start 153.035 116.3955) (end 148.59 111.9505) (width 0.25) (layer B.Cu) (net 8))
 (segment (start 148.59 111.9505) (end 148.59 111.533) (width 0.25) (layer B.Cu) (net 8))
 (segment (start 149.86 120.65) (end 150.2505 120.65) (width 0.25) (layer B.Cu) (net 10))
 (segment (start 152.4 118.5005) (end 152.4 118.083) (width 0.25) (layer B.Cu) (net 10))
 (segment (start 150.2505 120.65) (end 152.4 118.5005) (width 0.25) (layer B.Cu) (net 10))
 (segment (start 147.32 120.65) (end 147.32 120.269) (width 0.25) (layer B.Cu) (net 11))
 (segment (start 147.32 120.269) (end 148.5845 119.0045) (width 0.25) (layer B.Cu) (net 11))
 (segment (start 148.5845 119.0045) (end 148.59 119.0045) (width 0.25) (layer B.Cu) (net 11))
 (segment (start 148.59 119.0045) (end 148.59 118.083) (width 0.25) (layer B.Cu) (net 11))
 (segment (start 144.78 120.65) (end 144.78 120.4976) (width 0.25) (layer B.Cu) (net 7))
 (segment (start 144.78 120.4976) (end 145.415 119.8626) (width 0.25) (layer B.Cu) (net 7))
 (segment (start 145.415 119.8626) (end 145.415 112.9665) (width 0.25) (layer B.Cu) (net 7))
 (segment (start 144.78 112.3315) (end 144.78 111.533) (width 0.25) (layer B.Cu) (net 7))
 (segment (start 145.415 112.9665) (end 144.78 112.3315) (width 0.25) (layer B.Cu) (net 7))
 (segment (start 147.32 109.728) (end 147.367 109.775) (width 0.25) (layer B.Cu) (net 1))
 (segment (start 147.367 109.775) (end 154.04 109.775) (width 0.25) (layer B.Cu) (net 1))
 (segment (start 154.04 109.775) (end 154.94 109.775) (width 0.25) (layer B.Cu) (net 1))
 (via (at 147.32 109.728) (size 0.6) (drill 0.4) (layers F.Cu B.Cu) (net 1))
 (segment (start 147.32 109.728) (end 147.32 105.41) (width 0.25) (layer F.Cu) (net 1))
 (segment (start 147.32 109.728) (end 146.812 109.728) (width 0.25) (layer F.Cu) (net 1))
 (segment (start 146.812 109.728) (end 146.05 110.49) (width 0.25) (layer F.Cu) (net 1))
 (segment (start 146.558 109.728) (end 146.05 110.236) (width 0.25) (layer B.Cu) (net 1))
 (segment (start 146.05 110.49) (end 145.49 110.49) (width 0.25) (layer F.Cu) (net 1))
 (segment (start 147.32 109.728) (end 146.558 109.728) (width 0.25) (layer B.Cu) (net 1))
 (segment (start 146.05 110.236) (end 146.05 111.533) (width 0.25) (layer B.Cu) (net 1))
 (segment (start 147.32 102.87) (end 148.59 104.14) (width 0.25) (layer F.Cu) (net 6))
 (segment (start 148.59 104.14) (end 148.59 112.903) (width 0.25) (layer F.Cu) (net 6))
 (segment (start 148.59 112.903) (end 148.590006 112.903) (width 0.25) (layer F.Cu) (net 6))
 (segment (start 148.590006 112.903) (end 148.717006 113.03) (width 0.25) (layer F.Cu) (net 6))
 (segment (start 148.3995 113.03) (end 148.717006 113.03) (width 0.25) (layer B.Cu) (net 6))
 (segment (start 147.32 111.9505) (end 148.3995 113.03) (width 0.25) (layer B.Cu) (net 6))
 (segment (start 147.32 111.533) (end 147.32 111.9505) (width 0.25) (layer B.Cu) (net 6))
 (segment (start 151.69 113.03) (end 148.717006 113.03) (width 0.25) (layer F.Cu) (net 6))
 (via (at 148.717006 113.03) (size 0.6) (drill 0.4) (layers F.Cu B.Cu) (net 6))
 (segment (start 151.429999 115.206501) (end 151.13 115.5065) (width 0.25) (layer F.Cu) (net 5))
 (segment (start 151.69 114.9465) (end 151.429999 115.206501) (width 0.25) (layer F.Cu) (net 5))
 (segment (start 151.69 114.3) (end 151.69 114.9465) (width 0.25) (layer F.Cu) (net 5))
 (segment (start 151.13 118.083) (end 151.13 115.5065) (width 0.25) (layer B.Cu) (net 5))
 (via (at 151.13 115.5065) (size 0.6) (drill 0.4) (layers F.Cu B.Cu) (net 5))
 (segment (start 151.69 114.3) (end 153.115 114.3) (width 0.25) (layer F.Cu) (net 5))
 (segment (start 153.115 114.3) (end 153.543 113.872) (width 0.25) (layer F.Cu) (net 5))
 (segment (start 153.543 113.872) (end 153.543 113.03) (width 0.25) (layer F.Cu) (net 5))
 (segment (start 153.543 113.03) (end 154.168001 112.404999) (width 0.25) (layer F.Cu) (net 5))
 (segment (start 154.168001 109.718001) (end 149.86 105.41) (width 0.25) (layer F.Cu) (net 5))
 (segment (start 154.168001 112.404999) (end 154.168001 109.718001) (width 0.25) (layer F.Cu) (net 5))
 (segment (start 146.177 106.553) (end 146.177 106.649087) (width 0.25) (layer F.Cu) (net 2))
 (segment (start 146.177 106.649087) (end 143.891 108.935087) (width 0.25) (layer F.Cu) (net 2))
 (segment (start 143.891 108.935087) (end 143.891 111.252) (width 0.25) (layer F.Cu) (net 2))
 (segment (start 143.891 111.252) (end 144.399 111.76) (width 0.25) (layer F.Cu) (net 2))
 (segment (start 144.399 111.76) (end 145.49 111.76) (width 0.25) (layer F.Cu) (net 2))
 (segment (start 146.177 106.553) (end 146.05 106.426) (width 0.25) (layer B.Cu) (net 2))
 (segment (start 146.05 106.426) (end 146.05 104.648) (width 0.25) (layer B.Cu) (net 2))
 (segment (start 146.05 104.648) (end 146.558 104.14) (width 0.25) (layer B.Cu) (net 2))
 (segment (start 146.558 104.14) (end 148.59 104.14) (width 0.25) (layer B.Cu) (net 2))
 (segment (start 148.59 104.14) (end 149.86 102.87) (width 0.25) (layer B.Cu) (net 2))
 (via (at 146.177 106.553) (size 0.6) (drill 0.4) (layers F.Cu B.Cu) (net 2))
 (segment (start 149.86 115.255) (end 149.86 115.6335) (width 0.25) (layer F.Cu) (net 2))
 (segment (start 146.365 111.76) (end 149.86 115.255) (width 0.25) (layer F.Cu) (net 2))
 (segment (start 145.49 111.76) (end 146.365 111.76) (width 0.25) (layer F.Cu) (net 2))
 (segment (start 149.86 118.083) (end 149.86 115.6335) (width 0.25) (layer B.Cu) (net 2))
 (via (at 149.86 115.6335) (size 0.6) (drill 0.4) (layers F.Cu B.Cu) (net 2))
 (segment (start 151.13 111.533) (end 151.13 110.871) (width 0.25) (layer B.Cu) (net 9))
 (segment (start 151.13 110.871) (end 151.638 110.363) (width 0.25) (layer B.Cu) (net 9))
 (segment (start 151.638 110.363) (end 153.162 110.363) (width 0.25) (layer B.Cu) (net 9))
 (segment (start 153.162 110.363) (end 153.924 111.125) (width 0.25) (layer B.Cu) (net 9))
 (segment (start 153.924 111.125) (end 155.829 111.125) (width 0.25) (layer B.Cu) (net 9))
 (segment (start 155.829 111.125) (end 156.083 110.871) (width 0.25) (layer B.Cu) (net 9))
 (segment (start 156.083 110.871) (end 156.083 104.775) (width 0.25) (layer B.Cu) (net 9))
 (segment (start 156.083 104.775) (end 154.178 102.87) (width 0.25) (layer B.Cu) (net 9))
 (segment (start 154.178 102.87) (end 152.4 102.87) (width 0.25) (layer B.Cu) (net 9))
 (segment (start 147.32 118.083) (end 147.32 117.1615) (width 0.25) (layer B.Cu) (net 9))
 (segment (start 147.32 117.1615) (end 146.685 116.5265) (width 0.25) (layer B.Cu) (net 9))
 (segment (start 146.685 116.5265) (end 146.685 110.617) (width 0.25) (layer B.Cu) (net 9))
 (segment (start 146.685 110.617) (end 146.939 110.363) (width 0.25) (layer B.Cu) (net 9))
 (segment (start 146.939 110.363) (end 149.352 110.363) (width 0.25) (layer B.Cu) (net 9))
 (segment (start 149.352 110.363) (end 149.86 110.871) (width 0.25) (layer B.Cu) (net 9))
 (segment (start 149.86 110.871) (end 149.86 111.533) (width 0.25) (layer B.Cu) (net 9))
 (segment (start 152.4 102.87) (end 151.13 104.14) (width 0.25) (layer B.Cu) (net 9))
 (segment (start 151.13 104.14) (end 151.13 106.553) (width 0.25) (layer B.Cu) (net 9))
 (segment (start 151.13 106.553) (end 150.495 107.188) (width 0.25) (layer B.Cu) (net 9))
 (segment (start 150.495 107.188) (end 145.796 107.188) (width 0.25) (layer B.Cu) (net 9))
 (segment (start 145.796 107.188) (end 143.209 109.775) (width 0.25) (layer B.Cu) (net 9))
 (segment (start 143.209 109.775) (end 143.14 109.775) (width 0.25) (layer B.Cu) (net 9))
 (segment (start 143.14 109.775) (end 142.24 109.775) (width 0.25) (layer B.Cu) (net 9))
 (segment (start 149.86 111.533) (end 151.13 111.533) (width 0.25) (layer B.Cu) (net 9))
 (segment (start 147.32 118.083) (end 146.05 118.083) (width 0.25) (layer B.Cu) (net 9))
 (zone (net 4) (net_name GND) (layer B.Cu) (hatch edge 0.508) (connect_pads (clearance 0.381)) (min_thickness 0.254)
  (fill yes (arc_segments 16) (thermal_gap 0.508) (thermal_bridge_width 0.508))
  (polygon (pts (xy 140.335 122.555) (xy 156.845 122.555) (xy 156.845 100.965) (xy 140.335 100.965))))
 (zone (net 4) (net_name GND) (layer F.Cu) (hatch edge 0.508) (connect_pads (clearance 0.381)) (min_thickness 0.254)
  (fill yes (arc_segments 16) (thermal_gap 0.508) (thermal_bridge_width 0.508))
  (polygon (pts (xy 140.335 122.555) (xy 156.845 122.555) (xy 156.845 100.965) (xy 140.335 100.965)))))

